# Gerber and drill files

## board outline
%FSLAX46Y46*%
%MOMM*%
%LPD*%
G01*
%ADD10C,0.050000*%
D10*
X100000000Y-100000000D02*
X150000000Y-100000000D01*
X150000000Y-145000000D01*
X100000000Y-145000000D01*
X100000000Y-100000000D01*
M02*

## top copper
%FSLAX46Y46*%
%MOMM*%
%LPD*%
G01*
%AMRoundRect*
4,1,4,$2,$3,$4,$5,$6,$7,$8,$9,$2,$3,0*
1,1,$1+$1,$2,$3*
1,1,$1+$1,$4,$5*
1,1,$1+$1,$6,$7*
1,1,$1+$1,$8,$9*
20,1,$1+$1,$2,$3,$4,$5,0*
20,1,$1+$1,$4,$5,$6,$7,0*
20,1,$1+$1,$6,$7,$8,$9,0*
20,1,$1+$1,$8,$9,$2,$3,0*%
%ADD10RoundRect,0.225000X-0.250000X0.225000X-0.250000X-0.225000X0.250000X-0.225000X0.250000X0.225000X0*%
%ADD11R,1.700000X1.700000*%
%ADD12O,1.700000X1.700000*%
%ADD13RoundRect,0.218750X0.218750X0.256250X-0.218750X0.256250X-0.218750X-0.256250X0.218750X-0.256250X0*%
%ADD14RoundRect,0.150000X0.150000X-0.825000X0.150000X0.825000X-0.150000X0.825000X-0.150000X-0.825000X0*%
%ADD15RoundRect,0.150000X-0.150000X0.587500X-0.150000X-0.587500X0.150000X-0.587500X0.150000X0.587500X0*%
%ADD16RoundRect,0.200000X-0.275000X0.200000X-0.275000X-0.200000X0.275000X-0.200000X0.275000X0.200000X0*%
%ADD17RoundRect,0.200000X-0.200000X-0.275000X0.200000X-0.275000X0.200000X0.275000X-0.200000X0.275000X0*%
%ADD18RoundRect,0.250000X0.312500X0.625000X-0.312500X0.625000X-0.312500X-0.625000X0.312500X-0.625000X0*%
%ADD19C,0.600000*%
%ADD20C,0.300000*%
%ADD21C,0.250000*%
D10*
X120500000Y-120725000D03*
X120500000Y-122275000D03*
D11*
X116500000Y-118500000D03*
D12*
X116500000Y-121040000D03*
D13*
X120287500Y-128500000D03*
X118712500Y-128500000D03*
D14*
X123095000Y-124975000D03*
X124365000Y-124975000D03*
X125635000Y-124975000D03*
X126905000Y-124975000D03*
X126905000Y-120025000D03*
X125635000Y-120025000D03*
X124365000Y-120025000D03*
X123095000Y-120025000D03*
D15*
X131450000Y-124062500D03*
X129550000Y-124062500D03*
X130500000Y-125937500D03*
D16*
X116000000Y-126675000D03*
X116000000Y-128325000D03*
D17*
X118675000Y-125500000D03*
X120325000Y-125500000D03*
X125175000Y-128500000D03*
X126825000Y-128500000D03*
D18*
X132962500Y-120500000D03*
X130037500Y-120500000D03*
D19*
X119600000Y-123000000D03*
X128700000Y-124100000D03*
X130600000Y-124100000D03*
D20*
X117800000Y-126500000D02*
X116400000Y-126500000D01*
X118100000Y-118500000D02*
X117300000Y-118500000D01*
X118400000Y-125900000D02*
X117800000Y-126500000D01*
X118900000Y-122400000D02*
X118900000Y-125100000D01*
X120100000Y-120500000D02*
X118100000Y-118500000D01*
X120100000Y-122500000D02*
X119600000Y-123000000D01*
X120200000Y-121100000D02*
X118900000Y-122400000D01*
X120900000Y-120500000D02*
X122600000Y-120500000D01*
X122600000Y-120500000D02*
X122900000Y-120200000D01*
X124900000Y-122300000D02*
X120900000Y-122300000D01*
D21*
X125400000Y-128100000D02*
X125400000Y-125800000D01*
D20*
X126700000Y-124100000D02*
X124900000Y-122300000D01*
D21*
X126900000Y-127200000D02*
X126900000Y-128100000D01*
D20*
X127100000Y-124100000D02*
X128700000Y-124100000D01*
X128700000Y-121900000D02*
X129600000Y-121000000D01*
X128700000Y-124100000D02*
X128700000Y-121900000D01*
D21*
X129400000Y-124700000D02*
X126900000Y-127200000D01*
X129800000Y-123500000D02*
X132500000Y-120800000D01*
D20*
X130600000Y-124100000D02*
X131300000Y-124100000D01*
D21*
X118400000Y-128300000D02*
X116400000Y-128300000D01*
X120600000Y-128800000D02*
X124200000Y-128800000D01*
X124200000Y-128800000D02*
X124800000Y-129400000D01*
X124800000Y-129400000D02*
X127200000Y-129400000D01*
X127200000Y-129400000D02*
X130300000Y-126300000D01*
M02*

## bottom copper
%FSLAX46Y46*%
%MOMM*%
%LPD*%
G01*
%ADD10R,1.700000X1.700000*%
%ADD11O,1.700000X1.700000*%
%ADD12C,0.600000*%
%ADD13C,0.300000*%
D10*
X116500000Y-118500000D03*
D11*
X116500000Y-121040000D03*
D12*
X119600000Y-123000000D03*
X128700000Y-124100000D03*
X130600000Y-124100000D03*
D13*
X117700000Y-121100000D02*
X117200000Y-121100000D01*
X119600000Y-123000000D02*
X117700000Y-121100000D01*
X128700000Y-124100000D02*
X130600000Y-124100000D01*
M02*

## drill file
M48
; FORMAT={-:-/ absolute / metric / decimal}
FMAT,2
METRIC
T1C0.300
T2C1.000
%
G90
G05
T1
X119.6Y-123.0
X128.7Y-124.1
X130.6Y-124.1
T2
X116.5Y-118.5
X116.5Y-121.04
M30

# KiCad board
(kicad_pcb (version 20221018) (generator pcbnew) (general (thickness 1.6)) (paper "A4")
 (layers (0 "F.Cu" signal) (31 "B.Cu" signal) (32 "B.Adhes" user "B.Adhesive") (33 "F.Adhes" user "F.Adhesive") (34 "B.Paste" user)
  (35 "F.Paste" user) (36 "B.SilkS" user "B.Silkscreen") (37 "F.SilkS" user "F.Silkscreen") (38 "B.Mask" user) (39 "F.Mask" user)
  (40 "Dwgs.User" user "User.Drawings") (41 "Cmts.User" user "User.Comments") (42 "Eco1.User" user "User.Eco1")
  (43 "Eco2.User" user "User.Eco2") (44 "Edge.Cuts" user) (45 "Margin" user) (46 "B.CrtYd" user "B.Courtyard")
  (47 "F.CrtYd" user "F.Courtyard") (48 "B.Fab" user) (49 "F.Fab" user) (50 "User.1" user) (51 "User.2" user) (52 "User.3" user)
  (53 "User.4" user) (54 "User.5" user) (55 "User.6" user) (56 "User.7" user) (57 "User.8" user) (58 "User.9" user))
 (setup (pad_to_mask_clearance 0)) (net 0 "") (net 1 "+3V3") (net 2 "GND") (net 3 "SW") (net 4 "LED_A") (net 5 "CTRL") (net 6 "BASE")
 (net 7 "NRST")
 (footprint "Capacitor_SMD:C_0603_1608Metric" (layer "F.Cu") (at 120.5 121.5 -90)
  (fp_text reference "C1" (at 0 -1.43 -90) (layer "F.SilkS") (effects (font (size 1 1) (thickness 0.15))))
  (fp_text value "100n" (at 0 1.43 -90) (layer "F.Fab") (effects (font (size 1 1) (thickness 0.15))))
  (pad "1" smd roundrect (at -0.775 0 270) (size 0.9 0.95) (layers "F.Cu" "F.Paste" "F.Mask") (roundrect_rratio 0.25) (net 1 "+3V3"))
  (pad "2" smd roundrect (at 0.775 0 270) (size 0.9 0.95) (layers "F.Cu" "F.Paste" "F.Mask") (roundrect_rratio 0.25) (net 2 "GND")))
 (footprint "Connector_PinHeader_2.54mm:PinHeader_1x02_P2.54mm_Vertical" (layer "F.Cu") (at 116.5 118.5)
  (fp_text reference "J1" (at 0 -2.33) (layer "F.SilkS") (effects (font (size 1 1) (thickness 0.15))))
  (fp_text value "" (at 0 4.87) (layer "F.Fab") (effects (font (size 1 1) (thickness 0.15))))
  (pad "1" thru_hole rect (at 0 0) (size 1.7 1.7) (drill 1) (layers "*.Cu" "*.Mask") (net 1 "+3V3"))
  (pad "2" thru_hole oval (at 0 2.54) (size 1.7 1.7) (drill 1) (layers "*.Cu" "*.Mask") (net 2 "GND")))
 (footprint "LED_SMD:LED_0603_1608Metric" (layer "F.Cu") (at 119.5 128.5 180)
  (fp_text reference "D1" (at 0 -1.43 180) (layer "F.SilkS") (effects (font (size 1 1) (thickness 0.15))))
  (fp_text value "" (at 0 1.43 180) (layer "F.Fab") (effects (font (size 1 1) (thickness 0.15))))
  (pad "1" smd roundrect (at -0.7875 0 180) (size 0.875 0.95) (layers "F.Cu" "F.Paste" "F.Mask") (roundrect_rratio 0.25) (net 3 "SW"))
  (pad "2" smd roundrect (at 0.7875 0 180) (size 0.875 0.95) (layers "F.Cu" "F.Paste" "F.Mask") (roundrect_rratio 0.25) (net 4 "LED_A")))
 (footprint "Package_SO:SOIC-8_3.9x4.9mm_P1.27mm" (layer "F.Cu") (at 125 122.5 90)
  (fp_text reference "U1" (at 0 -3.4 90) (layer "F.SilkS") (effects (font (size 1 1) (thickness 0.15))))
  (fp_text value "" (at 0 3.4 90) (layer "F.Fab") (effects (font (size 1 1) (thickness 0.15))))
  (pad "1" smd roundrect (at -2.475 -1.905 90) (size 1.95 0.6) (layers "F.Cu" "F.Paste" "F.Mask") (roundrect_rratio 0.25))
  (pad "2" smd roundrect (at -2.475 -0.635 90) (size 1.95 0.6) (layers "F.Cu" "F.Paste" "F.Mask") (roundrect_rratio 0.25))
  (pad "3" smd roundrect (at -2.475 0.635 90) (size 1.95 0.6) (layers "F.Cu" "F.Paste" "F.Mask") (roundrect_rratio 0.25) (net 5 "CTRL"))
  (pad "4" smd roundrect (at -2.475 1.905 90) (size 1.95 0.6) (layers "F.Cu" "F.Paste" "F.Mask") (roundrect_rratio 0.25) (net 2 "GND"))
  (pad "5" smd roundrect (at 2.475 1.905 90) (size 1.95 0.6) (layers "F.Cu" "F.Paste" "F.Mask") (roundrect_rratio 0.25))
  (pad "6" smd roundrect (at 2.475 0.635 90) (size 1.95 0.6) (layers "F.Cu" "F.Paste" "F.Mask") (roundrect_rratio 0.25))
  (pad "7" smd roundrect (at 2.475 -0.635 90) (size 1.95 0.6) (layers "F.Cu" "F.Paste" "F.Mask") (roundrect_rratio 0.25))
  (pad "8" smd roundrect (at 2.475 -1.905 90) (size 1.95 0.6) (layers "F.Cu" "F.Paste" "F.Mask") (roundrect_rratio 0.25) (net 1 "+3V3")))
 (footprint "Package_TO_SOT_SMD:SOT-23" (layer "F.Cu") (at 130.5 125 -90)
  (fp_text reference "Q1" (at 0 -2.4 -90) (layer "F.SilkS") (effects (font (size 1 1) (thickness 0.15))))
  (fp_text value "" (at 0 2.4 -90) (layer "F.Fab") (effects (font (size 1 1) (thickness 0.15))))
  (pad "1" smd roundrect (at -0.9375 -0.95 270) (size 1.475 0.6) (layers "F.Cu" "F.Paste" "F.Mask") (roundrect_rratio 0.25) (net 2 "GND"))
  (pad "2" smd roundrect (at -0.9375 0.95 270) (size 1.475 0.6) (layers "F.Cu" "F.Paste" "F.Mask") (roundrect_rratio 0.25) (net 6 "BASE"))
  (pad "3" smd roundrect (at 0.9375 0 270) (size 1.475 0.6) (layers "F.Cu" "F.Paste" "F.Mask") (roundrect_rratio 0.25) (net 3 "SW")))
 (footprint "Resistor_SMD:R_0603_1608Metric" (layer "F.Cu") (at 116 127.5 -90)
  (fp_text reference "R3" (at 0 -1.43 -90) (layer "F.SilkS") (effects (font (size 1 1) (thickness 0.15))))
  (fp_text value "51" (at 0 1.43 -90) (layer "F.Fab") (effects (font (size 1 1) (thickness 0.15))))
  (pad "1" smd roundrect (at -0.825 0 270) (size 0.8 0.95) (layers "F.Cu" "F.Paste" "F.Mask") (roundrect_rratio 0.25) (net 1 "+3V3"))
  (pad "2" smd roundrect (at 0.825 0 270) (size 0.8 0.95) (layers "F.Cu" "F.Paste" "F.Mask") (roundrect_rratio 0.25) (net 4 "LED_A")))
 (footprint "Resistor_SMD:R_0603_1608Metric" (layer "F.Cu") (at 119.5 125.5)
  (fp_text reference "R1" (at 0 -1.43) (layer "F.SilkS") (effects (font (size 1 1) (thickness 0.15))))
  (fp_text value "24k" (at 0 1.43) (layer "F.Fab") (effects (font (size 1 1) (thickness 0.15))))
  (pad "1" smd roundrect (at -0.825 0) (size 0.8 0.95) (layers "F.Cu" "F.Paste" "F.Mask") (roundrect_rratio 0.25) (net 1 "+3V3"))
  (pad "2" smd roundrect (at 0.825 0) (size 0.8 0.95) (layers "F.Cu" "F.Paste" "F.Mask") (roundrect_rratio 0.25) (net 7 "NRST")))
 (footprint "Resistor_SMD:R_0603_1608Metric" (layer "F.Cu") (at 126 128.5)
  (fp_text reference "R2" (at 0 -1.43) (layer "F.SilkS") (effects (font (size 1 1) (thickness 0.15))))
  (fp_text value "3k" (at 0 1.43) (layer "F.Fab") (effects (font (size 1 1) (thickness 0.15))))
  (pad "1" smd roundrect (at -0.825 0) (size 0.8 0.95) (layers "F.Cu" "F.Paste" "F.Mask") (roundrect_rratio 0.25) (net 5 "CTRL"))
  (pad "2" smd roundrect (at 0.825 0) (size 0.8 0.95) (layers "F.Cu" "F.Paste" "F.Mask") (roundrect_rratio 0.25) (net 6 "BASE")))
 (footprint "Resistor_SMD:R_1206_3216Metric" (layer "F.Cu") (at 131.5 120.5 180)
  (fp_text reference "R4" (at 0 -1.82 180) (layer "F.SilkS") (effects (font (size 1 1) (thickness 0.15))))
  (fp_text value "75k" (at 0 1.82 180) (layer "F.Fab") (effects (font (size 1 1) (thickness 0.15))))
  (pad "1" smd roundrect (at -1.4625 0 180) (size 1.125 1.75) (layers "F.Cu" "F.Paste" "F.Mask") (roundrect_rratio 0.222222) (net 6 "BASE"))
  (pad "2" smd roundrect (at 1.4625 0 180) (size 1.125 1.75) (layers "F.Cu" "F.Paste" "F.Mask") (roundrect_rratio 0.222222) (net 2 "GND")))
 (gr_rect (start 100 100) (end 150 145) (stroke (width 0.05) (type default)) (fill none) (layer "Edge.Cuts"))
 (segment (start 117.8 126.5) (end 116.4 126.5) (width 0.3) (layer "F.Cu") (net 1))
 (segment (start 118.1 118.5) (end 117.3 118.5) (width 0.3) (layer "F.Cu") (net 1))
 (segment (start 118.4 125.9) (end 117.8 126.5) (width 0.3) (layer "F.Cu") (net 1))
 (segment (start 118.9 122.4) (end 118.9 125.1) (width 0.3) (layer "F.Cu") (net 1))
 (segment (start 120.1 120.5) (end 118.1 118.5) (width 0.3) (layer "F.Cu") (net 1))
 (segment (start 120.1 122.5) (end 119.6 123) (width 0.3) (layer "F.Cu") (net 2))
 (segment (start 120.2 121.1) (end 118.9 122.4) (width 0.3) (layer "F.Cu") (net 1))
 (segment (start 120.9 120.5) (end 122.6 120.5) (width 0.3) (layer "F.Cu") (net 1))
 (segment (start 122.6 120.5) (end 122.9 120.2) (width 0.3) (layer "F.Cu") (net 1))
 (segment (start 124.9 122.3) (end 120.9 122.3) (width 0.3) (layer "F.Cu") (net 2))
 (segment (start 125.4 128.1) (end 125.4 125.8) (width 0.25) (layer "F.Cu") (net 5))
 (segment (start 126.7 124.1) (end 124.9 122.3) (width 0.3) (layer "F.Cu") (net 2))
 (segment (start 126.9 127.2) (end 126.9 128.1) (width 0.25) (layer "F.Cu") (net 6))
 (segment (start 127.1 124.1) (end 128.7 124.1) (width 0.3) (layer "F.Cu") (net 2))
 (segment (start 128.7 121.9) (end 129.6 121) (width 0.3) (layer "F.Cu") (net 2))
 (segment (start 128.7 124.1) (end 128.7 121.9) (width 0.3) (layer "F.Cu") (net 2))
 (segment (start 129.4 124.7) (end 126.9 127.2) (width 0.25) (layer "F.Cu") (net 6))
 (segment (start 129.8 123.5) (end 132.5 120.8) (width 0.25) (layer "F.Cu") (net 6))
 (segment (start 130.6 124.1) (end 131.3 124.1) (width 0.3) (layer "F.Cu") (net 2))
 (via (at 119.6 123) (size 0.6) (drill 0.3) (layers "F.Cu" "B.Cu") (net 2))
 (via (at 128.7 124.1) (size 0.6) (drill 0.3) (layers "F.Cu" "B.Cu") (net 2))
 (via (at 130.6 124.1) (size 0.6) (drill 0.3) (layers "F.Cu" "B.Cu") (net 2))
 (segment (start 117.7 121.1) (end 117.2 121.1) (width 0.3) (layer "B.Cu") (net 2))
 (segment (start 118.4 128.3) (end 116.4 128.3) (width 0.25) (layer "F.Cu") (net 4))
 (segment (start 119.6 123) (end 117.7 121.1) (width 0.3) (layer "B.Cu") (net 2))
 (segment (start 120.6 128.8) (end 124.2 128.8) (width 0.25) (layer "F.Cu") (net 3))
 (segment (start 124.2 128.8) (end 124.8 129.4) (width 0.25) (layer "F.Cu") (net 3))
 (segment (start 124.8 129.4) (end 127.2 129.4) (width 0.25) (layer "F.Cu") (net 3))
 (segment (start 127.2 129.4) (end 130.3 126.3) (width 0.25) (layer "F.Cu") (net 3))
 (segment (start 128.7 124.1) (end 130.6 124.1) (width 0.3) (layer "B.Cu") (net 2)))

